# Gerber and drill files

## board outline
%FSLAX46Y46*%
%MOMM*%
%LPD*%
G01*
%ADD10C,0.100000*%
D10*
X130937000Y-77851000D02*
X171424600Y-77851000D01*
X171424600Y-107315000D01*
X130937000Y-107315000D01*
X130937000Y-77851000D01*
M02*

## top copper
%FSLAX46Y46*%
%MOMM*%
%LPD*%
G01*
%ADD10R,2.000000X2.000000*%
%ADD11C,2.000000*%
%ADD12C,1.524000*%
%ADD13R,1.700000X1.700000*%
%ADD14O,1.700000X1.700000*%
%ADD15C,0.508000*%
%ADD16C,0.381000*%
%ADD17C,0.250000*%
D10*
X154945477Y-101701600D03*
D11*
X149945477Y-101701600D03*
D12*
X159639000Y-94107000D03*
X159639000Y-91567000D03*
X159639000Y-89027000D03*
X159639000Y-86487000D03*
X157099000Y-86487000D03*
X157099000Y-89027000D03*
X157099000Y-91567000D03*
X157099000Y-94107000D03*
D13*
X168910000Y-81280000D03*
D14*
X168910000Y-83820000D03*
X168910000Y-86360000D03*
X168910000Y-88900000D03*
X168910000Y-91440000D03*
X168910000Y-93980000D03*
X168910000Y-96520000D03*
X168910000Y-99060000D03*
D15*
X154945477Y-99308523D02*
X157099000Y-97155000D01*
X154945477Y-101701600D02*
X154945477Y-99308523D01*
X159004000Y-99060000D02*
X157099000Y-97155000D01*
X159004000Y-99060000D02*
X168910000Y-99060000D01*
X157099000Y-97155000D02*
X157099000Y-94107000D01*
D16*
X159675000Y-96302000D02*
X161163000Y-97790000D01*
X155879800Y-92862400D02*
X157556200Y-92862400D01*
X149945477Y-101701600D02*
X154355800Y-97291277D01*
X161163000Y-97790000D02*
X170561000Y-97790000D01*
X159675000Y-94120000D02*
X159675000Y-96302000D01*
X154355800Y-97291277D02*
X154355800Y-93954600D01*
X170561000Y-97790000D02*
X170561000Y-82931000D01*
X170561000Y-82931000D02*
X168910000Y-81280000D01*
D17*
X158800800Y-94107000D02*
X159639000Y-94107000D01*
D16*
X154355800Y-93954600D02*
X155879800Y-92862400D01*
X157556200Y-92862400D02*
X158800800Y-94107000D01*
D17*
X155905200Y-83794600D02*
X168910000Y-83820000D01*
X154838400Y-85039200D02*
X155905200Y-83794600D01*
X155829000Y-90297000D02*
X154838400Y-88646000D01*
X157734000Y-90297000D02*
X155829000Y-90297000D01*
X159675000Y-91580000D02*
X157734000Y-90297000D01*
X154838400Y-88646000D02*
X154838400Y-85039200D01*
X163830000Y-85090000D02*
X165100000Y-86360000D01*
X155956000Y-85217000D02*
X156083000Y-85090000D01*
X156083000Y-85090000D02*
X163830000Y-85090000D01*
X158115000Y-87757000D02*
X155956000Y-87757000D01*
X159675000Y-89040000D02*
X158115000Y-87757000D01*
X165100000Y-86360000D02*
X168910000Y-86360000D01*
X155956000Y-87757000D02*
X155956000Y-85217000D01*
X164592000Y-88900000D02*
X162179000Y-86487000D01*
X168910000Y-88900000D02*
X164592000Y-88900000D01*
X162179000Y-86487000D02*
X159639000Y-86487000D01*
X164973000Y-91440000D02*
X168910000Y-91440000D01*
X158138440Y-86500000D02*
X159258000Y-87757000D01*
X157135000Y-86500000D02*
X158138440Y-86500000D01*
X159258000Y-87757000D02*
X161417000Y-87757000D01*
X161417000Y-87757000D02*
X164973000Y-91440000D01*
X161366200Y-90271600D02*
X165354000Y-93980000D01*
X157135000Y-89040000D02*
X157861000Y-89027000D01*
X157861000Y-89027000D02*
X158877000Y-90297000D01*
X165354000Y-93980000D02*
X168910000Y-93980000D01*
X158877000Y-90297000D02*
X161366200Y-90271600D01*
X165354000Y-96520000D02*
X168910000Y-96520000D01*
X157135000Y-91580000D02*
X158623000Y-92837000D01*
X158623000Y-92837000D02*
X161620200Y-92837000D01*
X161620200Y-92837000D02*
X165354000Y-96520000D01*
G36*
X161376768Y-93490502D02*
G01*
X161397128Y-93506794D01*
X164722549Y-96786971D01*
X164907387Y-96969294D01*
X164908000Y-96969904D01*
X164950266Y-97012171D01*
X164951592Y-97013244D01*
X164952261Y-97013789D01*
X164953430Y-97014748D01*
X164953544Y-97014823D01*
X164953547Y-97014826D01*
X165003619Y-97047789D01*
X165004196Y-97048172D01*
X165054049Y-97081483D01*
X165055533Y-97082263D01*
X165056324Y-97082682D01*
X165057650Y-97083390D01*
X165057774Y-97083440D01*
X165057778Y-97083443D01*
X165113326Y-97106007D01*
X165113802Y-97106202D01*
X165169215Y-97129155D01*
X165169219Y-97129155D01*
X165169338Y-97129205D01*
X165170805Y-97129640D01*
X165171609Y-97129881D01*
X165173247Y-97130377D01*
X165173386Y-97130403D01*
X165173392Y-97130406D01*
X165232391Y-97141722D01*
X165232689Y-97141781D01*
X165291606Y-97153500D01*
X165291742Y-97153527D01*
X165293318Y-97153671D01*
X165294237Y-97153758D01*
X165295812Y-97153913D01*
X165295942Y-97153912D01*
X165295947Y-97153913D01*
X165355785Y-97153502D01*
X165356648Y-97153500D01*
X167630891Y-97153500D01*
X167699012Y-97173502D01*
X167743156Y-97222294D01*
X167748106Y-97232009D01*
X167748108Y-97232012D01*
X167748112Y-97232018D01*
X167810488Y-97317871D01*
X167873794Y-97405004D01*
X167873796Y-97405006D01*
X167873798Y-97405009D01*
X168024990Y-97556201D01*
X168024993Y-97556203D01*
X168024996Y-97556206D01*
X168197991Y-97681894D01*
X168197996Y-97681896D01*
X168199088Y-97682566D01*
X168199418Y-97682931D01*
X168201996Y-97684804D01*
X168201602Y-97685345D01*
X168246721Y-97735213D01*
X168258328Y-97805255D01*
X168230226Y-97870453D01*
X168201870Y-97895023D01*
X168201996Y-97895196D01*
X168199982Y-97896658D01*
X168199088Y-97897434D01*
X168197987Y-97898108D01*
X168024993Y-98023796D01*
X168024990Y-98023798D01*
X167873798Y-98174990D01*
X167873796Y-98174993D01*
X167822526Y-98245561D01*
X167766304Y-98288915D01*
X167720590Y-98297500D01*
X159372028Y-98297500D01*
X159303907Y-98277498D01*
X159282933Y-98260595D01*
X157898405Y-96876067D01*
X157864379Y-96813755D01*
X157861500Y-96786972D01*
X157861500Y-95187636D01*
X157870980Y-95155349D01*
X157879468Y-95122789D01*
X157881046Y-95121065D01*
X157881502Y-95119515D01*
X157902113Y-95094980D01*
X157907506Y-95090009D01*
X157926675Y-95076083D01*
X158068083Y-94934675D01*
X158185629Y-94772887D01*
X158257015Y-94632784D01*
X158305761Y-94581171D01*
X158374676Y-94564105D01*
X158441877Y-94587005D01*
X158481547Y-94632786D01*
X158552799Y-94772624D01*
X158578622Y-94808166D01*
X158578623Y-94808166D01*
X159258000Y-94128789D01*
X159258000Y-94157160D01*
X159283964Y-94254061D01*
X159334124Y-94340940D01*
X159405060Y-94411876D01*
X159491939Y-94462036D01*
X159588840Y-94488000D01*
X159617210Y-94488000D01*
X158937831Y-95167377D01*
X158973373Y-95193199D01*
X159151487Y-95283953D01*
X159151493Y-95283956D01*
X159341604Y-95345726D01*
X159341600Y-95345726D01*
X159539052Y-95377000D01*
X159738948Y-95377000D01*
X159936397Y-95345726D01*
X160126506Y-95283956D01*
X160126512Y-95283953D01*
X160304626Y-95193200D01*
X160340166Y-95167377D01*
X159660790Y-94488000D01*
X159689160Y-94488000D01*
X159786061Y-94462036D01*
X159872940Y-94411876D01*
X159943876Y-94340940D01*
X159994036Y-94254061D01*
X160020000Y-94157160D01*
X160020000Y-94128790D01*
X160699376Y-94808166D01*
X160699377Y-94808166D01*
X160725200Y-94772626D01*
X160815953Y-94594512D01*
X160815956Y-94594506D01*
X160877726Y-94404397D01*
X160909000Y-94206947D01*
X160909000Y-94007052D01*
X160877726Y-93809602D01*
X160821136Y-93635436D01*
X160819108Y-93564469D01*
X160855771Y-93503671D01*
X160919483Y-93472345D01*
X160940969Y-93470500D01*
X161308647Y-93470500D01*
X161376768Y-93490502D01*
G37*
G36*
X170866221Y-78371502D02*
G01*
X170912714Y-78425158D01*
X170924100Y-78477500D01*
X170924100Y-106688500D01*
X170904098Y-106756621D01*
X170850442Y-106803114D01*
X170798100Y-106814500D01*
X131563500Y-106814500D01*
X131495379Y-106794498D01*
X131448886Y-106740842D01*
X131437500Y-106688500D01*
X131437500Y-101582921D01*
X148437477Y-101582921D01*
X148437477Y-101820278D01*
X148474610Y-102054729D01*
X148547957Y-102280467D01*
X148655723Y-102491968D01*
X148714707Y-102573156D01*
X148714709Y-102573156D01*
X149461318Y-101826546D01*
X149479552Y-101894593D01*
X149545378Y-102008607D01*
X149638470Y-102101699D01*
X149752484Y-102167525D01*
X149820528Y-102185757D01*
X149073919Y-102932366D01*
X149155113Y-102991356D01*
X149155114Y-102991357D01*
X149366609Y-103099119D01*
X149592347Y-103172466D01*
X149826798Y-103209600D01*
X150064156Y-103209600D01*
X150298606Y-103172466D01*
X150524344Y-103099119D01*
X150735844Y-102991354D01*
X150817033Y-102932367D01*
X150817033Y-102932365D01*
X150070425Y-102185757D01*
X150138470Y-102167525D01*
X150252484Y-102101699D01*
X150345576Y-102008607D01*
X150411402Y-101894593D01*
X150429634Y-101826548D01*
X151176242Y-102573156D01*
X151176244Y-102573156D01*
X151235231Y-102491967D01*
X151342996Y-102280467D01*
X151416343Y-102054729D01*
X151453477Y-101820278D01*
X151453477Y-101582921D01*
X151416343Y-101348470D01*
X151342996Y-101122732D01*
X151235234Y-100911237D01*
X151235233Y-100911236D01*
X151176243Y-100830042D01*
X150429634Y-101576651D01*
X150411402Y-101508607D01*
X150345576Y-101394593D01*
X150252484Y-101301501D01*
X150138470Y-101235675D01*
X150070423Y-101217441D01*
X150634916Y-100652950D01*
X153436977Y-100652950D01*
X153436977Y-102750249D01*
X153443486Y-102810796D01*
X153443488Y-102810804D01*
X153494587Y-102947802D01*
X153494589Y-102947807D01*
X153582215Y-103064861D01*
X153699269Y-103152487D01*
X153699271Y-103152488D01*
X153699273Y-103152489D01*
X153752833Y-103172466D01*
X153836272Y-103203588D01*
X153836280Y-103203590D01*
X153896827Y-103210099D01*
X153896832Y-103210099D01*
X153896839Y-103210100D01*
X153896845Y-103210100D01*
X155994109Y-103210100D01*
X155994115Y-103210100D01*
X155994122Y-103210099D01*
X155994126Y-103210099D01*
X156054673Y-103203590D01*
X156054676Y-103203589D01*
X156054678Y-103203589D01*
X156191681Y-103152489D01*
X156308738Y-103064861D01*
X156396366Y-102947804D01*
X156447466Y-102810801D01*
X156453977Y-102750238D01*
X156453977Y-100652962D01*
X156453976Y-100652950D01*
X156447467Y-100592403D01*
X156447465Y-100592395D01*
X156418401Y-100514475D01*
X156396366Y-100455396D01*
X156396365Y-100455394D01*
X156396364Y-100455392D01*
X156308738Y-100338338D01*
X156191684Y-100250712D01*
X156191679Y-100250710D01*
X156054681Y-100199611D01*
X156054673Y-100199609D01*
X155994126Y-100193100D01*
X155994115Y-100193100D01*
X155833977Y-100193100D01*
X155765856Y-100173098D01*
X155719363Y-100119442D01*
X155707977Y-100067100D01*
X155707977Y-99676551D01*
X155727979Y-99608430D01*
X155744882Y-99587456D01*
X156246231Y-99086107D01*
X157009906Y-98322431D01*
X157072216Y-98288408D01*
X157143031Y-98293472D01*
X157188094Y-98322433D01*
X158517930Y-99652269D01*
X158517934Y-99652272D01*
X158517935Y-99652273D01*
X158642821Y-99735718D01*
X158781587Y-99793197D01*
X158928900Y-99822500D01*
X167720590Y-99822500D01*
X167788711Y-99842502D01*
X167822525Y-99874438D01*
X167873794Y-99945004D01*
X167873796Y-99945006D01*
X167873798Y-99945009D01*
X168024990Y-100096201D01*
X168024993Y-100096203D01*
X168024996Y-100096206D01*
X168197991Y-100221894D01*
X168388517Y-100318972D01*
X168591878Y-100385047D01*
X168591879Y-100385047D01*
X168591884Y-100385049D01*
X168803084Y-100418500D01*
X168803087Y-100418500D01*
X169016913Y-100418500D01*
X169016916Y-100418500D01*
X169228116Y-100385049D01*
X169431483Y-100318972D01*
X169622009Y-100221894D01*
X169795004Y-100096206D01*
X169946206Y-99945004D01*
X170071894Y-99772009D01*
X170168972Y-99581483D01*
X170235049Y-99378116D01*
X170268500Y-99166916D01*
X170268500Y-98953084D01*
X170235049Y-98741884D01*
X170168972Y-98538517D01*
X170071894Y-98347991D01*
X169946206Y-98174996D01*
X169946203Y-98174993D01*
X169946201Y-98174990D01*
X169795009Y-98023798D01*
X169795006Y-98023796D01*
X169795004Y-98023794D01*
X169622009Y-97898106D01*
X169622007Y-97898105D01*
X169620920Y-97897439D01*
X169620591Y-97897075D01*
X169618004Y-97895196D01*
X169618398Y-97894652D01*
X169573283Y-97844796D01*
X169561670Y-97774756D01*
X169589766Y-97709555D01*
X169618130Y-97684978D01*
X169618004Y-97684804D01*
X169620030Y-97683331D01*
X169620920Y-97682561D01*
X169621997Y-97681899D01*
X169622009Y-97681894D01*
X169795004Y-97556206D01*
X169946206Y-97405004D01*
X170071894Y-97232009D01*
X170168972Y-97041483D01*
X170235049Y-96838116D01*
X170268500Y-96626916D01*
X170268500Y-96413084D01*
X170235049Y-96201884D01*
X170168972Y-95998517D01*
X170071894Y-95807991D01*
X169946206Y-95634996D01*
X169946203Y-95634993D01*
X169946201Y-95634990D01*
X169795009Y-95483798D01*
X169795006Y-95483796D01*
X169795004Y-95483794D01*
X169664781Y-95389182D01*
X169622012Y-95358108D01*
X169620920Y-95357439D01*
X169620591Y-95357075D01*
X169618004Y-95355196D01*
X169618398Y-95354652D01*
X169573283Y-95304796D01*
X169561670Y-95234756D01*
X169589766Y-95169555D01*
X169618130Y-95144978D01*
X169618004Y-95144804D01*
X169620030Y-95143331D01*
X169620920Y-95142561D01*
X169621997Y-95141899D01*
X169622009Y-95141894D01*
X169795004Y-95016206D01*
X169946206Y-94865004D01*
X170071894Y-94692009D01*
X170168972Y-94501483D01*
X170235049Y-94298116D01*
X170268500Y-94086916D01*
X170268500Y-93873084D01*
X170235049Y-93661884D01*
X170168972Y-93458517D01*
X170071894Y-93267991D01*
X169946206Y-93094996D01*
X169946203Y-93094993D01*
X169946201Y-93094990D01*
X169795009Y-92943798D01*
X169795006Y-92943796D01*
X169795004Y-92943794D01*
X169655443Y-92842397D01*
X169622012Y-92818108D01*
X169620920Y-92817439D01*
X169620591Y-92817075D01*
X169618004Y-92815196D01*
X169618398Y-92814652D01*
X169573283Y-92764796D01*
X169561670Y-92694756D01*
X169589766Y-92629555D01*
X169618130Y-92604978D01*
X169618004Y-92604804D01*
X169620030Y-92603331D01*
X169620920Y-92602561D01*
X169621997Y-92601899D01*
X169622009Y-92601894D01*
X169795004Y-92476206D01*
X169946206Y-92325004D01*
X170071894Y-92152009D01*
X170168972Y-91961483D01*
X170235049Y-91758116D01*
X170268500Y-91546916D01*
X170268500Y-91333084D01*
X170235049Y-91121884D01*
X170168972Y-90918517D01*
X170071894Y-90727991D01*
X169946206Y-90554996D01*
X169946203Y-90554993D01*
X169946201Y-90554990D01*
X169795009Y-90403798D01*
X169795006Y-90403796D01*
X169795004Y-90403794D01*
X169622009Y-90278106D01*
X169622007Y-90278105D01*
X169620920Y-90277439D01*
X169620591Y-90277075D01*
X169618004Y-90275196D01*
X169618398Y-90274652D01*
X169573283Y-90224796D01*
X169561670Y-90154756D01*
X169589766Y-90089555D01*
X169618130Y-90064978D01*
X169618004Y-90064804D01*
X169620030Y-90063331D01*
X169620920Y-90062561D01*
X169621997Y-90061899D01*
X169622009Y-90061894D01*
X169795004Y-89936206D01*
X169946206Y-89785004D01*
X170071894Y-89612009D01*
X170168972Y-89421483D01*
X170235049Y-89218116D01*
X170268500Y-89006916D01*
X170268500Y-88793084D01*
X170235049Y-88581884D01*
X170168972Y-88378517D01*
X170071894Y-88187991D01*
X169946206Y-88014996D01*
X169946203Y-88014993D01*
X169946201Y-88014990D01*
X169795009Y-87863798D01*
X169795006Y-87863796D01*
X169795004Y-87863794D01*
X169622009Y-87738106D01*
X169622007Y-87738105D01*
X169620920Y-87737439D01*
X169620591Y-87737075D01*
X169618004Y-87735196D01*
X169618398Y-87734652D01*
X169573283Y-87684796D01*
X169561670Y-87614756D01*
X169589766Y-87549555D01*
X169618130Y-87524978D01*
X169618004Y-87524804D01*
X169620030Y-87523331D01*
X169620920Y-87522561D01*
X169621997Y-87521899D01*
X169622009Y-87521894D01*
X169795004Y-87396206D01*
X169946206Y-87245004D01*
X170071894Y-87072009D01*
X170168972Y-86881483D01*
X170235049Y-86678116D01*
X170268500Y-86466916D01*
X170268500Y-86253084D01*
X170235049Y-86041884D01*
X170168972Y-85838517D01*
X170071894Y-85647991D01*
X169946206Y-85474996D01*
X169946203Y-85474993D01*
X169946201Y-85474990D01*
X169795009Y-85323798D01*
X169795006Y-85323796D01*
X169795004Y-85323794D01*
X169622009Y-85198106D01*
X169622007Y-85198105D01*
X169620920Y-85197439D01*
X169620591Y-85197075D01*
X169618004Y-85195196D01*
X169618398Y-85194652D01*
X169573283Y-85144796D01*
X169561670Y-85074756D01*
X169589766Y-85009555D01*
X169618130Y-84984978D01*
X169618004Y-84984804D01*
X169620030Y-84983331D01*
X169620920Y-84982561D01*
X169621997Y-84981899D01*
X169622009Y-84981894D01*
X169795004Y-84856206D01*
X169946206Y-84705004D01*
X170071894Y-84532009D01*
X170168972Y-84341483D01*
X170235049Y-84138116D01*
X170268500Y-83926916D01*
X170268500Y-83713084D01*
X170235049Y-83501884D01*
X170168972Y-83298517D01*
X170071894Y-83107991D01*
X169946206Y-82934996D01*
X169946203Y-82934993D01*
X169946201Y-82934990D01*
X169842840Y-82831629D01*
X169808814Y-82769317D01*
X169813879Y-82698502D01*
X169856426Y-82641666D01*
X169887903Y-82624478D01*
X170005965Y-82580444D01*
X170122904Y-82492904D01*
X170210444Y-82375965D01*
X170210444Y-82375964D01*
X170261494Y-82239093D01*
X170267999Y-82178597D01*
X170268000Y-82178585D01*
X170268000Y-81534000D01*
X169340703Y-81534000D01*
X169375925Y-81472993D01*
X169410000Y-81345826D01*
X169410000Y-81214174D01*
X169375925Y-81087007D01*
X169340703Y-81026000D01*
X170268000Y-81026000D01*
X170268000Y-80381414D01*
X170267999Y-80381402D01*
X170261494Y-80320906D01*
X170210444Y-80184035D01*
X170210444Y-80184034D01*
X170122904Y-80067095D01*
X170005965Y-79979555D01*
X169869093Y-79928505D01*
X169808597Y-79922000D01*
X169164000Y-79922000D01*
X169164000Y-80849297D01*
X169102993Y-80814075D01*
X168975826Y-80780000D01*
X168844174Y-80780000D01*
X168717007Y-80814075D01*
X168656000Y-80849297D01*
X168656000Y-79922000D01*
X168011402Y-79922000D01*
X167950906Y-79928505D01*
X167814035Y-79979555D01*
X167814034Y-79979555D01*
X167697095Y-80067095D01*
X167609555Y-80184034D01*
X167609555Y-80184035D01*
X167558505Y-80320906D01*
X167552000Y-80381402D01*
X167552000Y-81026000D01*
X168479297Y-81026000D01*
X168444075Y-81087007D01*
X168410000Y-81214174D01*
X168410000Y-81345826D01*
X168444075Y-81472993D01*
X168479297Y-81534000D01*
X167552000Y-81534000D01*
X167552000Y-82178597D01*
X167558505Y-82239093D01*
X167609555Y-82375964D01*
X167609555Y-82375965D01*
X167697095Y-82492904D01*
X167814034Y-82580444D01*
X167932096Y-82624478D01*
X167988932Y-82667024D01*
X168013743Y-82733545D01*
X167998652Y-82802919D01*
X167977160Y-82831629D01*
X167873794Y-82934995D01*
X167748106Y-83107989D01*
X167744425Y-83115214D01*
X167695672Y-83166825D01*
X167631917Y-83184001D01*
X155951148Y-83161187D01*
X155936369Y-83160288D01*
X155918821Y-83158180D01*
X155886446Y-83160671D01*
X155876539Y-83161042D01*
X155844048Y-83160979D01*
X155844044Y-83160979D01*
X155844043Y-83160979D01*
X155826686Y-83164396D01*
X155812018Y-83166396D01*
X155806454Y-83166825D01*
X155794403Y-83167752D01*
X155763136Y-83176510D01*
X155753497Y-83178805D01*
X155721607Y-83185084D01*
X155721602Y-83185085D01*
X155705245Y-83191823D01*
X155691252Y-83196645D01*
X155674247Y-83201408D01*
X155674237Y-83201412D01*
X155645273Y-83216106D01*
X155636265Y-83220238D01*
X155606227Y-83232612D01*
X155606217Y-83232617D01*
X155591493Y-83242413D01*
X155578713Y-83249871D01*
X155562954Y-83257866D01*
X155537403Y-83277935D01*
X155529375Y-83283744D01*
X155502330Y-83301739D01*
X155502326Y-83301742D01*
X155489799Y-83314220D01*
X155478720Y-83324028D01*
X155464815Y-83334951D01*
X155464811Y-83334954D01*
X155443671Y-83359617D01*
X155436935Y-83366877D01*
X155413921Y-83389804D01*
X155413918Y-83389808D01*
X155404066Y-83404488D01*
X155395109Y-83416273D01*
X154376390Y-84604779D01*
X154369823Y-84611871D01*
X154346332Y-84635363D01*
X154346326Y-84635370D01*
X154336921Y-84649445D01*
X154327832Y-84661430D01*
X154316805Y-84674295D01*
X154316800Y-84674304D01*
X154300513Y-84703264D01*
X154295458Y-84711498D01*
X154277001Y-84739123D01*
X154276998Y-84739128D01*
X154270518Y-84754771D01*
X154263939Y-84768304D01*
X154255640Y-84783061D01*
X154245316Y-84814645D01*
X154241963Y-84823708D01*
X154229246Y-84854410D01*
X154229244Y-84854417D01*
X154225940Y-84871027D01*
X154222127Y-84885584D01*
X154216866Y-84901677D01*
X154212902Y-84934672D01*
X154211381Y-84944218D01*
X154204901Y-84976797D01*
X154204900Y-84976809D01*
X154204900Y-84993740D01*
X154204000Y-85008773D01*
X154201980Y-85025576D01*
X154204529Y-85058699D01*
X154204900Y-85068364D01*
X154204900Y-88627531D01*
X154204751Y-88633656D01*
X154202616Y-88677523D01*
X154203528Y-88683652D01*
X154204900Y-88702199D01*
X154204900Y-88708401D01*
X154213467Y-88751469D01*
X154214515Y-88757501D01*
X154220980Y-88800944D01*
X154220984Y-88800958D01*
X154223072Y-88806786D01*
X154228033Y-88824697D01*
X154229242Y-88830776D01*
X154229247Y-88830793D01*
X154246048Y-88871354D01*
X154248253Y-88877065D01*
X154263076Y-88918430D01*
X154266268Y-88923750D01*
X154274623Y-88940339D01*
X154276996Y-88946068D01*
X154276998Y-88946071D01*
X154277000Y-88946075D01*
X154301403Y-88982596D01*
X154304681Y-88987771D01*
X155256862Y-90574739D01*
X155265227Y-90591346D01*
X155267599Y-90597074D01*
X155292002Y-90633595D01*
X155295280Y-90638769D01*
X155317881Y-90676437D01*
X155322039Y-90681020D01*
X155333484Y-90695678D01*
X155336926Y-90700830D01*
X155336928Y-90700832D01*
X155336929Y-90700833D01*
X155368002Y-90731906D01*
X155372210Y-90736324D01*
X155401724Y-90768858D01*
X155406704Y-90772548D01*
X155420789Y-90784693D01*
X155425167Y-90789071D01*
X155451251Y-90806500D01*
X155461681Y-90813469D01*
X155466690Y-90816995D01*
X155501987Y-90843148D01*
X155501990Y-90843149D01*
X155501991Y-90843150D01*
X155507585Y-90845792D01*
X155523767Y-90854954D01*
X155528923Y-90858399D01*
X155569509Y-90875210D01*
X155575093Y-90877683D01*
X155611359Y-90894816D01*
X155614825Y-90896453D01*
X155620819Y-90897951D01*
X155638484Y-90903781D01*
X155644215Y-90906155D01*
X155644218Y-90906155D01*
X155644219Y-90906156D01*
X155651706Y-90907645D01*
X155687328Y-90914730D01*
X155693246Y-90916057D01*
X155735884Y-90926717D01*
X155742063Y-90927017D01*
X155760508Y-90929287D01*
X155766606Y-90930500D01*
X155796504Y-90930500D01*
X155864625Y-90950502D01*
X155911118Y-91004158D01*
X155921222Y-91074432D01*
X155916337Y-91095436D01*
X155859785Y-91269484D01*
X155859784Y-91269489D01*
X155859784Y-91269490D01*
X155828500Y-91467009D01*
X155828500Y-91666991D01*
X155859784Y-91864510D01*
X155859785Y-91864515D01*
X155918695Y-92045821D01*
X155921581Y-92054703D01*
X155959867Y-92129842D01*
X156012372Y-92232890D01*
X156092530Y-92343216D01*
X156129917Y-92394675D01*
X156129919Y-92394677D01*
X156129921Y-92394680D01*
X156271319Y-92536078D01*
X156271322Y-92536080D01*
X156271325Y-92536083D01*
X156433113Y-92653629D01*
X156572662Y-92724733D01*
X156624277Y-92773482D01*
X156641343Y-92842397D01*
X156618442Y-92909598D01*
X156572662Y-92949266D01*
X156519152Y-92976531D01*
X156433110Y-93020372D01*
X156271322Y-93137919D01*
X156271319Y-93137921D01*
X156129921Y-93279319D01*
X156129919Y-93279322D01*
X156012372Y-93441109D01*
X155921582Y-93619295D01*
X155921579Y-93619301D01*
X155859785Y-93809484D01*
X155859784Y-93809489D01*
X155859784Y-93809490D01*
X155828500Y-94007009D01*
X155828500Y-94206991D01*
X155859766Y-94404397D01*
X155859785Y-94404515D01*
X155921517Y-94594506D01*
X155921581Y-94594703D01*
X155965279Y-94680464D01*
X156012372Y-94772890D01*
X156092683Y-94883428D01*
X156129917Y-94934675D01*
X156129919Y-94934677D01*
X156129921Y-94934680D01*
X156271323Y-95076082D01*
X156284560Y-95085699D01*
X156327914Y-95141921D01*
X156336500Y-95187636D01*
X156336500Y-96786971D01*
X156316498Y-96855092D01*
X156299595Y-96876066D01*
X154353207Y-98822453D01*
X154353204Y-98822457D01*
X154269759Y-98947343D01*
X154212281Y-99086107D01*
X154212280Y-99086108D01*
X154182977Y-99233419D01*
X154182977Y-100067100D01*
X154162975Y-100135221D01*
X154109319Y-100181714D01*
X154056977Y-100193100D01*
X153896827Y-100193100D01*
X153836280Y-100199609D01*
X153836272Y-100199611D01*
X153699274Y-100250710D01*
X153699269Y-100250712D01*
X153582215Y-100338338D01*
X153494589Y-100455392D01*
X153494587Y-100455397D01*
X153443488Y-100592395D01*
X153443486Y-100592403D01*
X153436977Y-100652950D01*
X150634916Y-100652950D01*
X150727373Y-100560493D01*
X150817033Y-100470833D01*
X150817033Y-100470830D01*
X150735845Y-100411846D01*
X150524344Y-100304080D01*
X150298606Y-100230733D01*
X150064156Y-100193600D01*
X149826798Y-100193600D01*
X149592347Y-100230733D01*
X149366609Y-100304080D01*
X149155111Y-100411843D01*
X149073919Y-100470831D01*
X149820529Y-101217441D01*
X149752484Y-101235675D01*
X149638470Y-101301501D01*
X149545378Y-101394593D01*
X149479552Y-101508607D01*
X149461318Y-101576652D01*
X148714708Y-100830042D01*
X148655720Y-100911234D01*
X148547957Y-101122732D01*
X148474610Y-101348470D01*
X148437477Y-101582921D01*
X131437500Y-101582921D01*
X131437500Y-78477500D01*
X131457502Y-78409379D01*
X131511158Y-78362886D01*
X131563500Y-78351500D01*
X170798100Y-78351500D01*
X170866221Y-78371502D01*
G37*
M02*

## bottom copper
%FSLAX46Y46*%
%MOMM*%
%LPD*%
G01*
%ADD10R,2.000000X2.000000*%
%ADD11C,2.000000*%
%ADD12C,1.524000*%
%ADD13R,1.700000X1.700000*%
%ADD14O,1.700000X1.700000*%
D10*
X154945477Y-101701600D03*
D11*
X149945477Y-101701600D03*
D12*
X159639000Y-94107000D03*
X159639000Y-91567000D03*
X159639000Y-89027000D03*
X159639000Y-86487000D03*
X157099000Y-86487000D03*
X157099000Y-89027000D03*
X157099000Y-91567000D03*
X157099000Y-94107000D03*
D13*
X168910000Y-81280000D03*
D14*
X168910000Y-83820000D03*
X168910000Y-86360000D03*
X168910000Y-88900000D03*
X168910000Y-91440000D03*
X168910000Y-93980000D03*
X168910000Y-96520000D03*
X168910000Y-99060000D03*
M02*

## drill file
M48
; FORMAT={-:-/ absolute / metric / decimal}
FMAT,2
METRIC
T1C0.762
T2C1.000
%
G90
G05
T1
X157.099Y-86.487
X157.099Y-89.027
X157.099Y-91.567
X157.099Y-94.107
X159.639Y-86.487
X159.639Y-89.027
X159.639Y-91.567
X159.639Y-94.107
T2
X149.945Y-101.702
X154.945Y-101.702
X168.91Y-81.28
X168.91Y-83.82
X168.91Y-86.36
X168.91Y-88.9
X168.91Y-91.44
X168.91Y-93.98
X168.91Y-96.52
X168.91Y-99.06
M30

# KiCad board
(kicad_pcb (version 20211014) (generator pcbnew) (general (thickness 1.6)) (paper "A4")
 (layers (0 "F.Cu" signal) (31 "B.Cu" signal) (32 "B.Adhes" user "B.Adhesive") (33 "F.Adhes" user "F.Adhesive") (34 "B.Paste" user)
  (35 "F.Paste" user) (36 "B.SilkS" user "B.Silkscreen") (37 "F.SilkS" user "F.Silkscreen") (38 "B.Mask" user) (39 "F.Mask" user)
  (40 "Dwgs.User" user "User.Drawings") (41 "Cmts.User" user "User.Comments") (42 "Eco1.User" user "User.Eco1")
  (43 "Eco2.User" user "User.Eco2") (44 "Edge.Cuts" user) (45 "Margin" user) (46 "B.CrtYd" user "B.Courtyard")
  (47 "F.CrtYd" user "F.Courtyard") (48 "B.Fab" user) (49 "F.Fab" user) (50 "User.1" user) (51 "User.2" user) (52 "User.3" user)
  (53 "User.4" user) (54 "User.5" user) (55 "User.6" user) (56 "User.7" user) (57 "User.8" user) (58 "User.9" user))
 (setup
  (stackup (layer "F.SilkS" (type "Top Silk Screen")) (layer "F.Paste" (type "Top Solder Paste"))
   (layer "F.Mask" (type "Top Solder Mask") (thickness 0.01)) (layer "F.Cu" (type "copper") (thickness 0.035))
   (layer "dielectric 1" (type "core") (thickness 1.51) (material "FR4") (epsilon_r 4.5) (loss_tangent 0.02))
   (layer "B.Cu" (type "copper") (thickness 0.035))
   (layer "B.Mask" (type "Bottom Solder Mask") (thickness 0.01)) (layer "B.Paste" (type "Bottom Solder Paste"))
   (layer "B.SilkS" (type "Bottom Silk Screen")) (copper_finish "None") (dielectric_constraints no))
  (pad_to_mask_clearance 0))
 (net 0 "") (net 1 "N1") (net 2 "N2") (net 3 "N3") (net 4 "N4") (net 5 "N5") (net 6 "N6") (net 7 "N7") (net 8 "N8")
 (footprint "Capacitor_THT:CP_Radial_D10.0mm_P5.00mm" (layer "F.Cu") (at 154.945477 101.7016 180)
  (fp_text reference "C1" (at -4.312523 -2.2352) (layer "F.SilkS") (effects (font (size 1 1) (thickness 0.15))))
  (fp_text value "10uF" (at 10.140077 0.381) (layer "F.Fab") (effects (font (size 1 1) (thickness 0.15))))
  (pad "1" thru_hole rect (at 0 0 180) (size 2 2) (drill 1) (layers *.Cu *.Mask) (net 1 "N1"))
  (pad "2" thru_hole circle (at 5 0 180) (size 2 2) (drill 1) (layers *.Cu *.Mask) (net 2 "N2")))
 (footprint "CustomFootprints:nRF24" (layer "F.Cu") (at 153.289 90.932)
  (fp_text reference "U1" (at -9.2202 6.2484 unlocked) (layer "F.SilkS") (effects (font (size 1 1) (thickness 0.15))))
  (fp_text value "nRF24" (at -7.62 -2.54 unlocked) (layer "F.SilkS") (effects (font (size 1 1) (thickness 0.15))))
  (pad "0" thru_hole circle (at 6.35 3.175) (size 1.524 1.524) (drill 0.762) (layers *.Cu *.Mask) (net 2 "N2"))
  (pad "1" thru_hole circle (at 6.35 0.635) (size 1.524 1.524) (drill 0.762) (layers *.Cu *.Mask) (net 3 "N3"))
  (pad "2" thru_hole circle (at 6.35 -1.905) (size 1.524 1.524) (drill 0.762) (layers *.Cu *.Mask) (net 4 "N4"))
  (pad "3" thru_hole circle (at 6.35 -4.445) (size 1.524 1.524) (drill 0.762) (layers *.Cu *.Mask) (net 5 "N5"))
  (pad "4" thru_hole circle (at 3.81 -4.445) (size 1.524 1.524) (drill 0.762) (layers *.Cu *.Mask) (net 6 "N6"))
  (pad "5" thru_hole circle (at 3.81 -1.905) (size 1.524 1.524) (drill 0.762) (layers *.Cu *.Mask) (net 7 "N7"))
  (pad "6" thru_hole circle (at 3.81 0.635) (size 1.524 1.524) (drill 0.762) (layers *.Cu *.Mask) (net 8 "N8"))
  (pad "7" thru_hole circle (at 3.81 3.175) (size 1.524 1.524) (drill 0.762) (layers *.Cu *.Mask) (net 1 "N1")))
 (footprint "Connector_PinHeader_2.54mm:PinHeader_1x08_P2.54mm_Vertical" (layer "B.Cu") (at 168.91 81.28 180)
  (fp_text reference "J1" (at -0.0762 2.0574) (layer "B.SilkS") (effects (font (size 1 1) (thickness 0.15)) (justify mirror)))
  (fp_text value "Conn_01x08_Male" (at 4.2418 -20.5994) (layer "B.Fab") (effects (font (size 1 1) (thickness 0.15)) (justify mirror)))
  (pad "1" thru_hole rect (at 0 0 180) (size 1.7 1.7) (drill 1) (layers *.Cu *.Mask) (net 2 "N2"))
  (pad "2" thru_hole oval (at 0 -2.54 180) (size 1.7 1.7) (drill 1) (layers *.Cu *.Mask) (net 3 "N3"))
  (pad "3" thru_hole oval (at 0 -5.08 180) (size 1.7 1.7) (drill 1) (layers *.Cu *.Mask) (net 4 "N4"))
  (pad "4" thru_hole oval (at 0 -7.62 180) (size 1.7 1.7) (drill 1) (layers *.Cu *.Mask) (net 5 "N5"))
  (pad "5" thru_hole oval (at 0 -10.16 180) (size 1.7 1.7) (drill 1) (layers *.Cu *.Mask) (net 6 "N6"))
  (pad "6" thru_hole oval (at 0 -12.7 180) (size 1.7 1.7) (drill 1) (layers *.Cu *.Mask) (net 7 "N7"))
  (pad "7" thru_hole oval (at 0 -15.24 180) (size 1.7 1.7) (drill 1) (layers *.Cu *.Mask) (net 8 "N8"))
  (pad "8" thru_hole oval (at 0 -17.78 180) (size 1.7 1.7) (drill 1) (layers *.Cu *.Mask) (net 1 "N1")))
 (gr_rect (start 130.937 77.851) (end 171.4246 107.315) (layer "Edge.Cuts") (width 0.1) (fill none))
 (segment (start 154.945477 99.308523) (end 157.099 97.155) (width 0.508) (layer "F.Cu") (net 1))
 (segment (start 154.945477 101.7016) (end 154.945477 99.308523) (width 0.508) (layer "F.Cu") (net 1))
 (segment (start 159.004 99.06) (end 157.099 97.155) (width 0.508) (layer "F.Cu") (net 1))
 (segment (start 159.004 99.06) (end 168.91 99.06) (width 0.508) (layer "F.Cu") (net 1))
 (segment (start 157.099 97.155) (end 157.099 94.107) (width 0.508) (layer "F.Cu") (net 1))
 (segment (start 159.675 96.302) (end 161.163 97.79) (width 0.381) (layer "F.Cu") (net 2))
 (segment (start 155.8798 92.8624) (end 157.5562 92.8624) (width 0.381) (layer "F.Cu") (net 2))
 (segment (start 149.945477 101.7016) (end 154.3558 97.291277) (width 0.381) (layer "F.Cu") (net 2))
 (segment (start 161.163 97.79) (end 170.561 97.79) (width 0.381) (layer "F.Cu") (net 2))
 (segment (start 159.675 94.12) (end 159.675 96.302) (width 0.381) (layer "F.Cu") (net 2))
 (segment (start 154.3558 97.291277) (end 154.3558 93.9546) (width 0.381) (layer "F.Cu") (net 2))
 (segment (start 170.561 97.79) (end 170.561 82.931) (width 0.381) (layer "F.Cu") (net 2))
 (segment (start 170.561 82.931) (end 168.91 81.28) (width 0.381) (layer "F.Cu") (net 2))
 (segment (start 158.8008 94.107) (end 159.639 94.107) (width 0.25) (layer "F.Cu") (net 2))
 (segment (start 154.3558 93.9546) (end 155.8798 92.8624) (width 0.381) (layer "F.Cu") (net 2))
 (segment (start 157.5562 92.8624) (end 158.8008 94.107) (width 0.381) (layer "F.Cu") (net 2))
 (segment (start 155.9052 83.7946) (end 168.91 83.82) (width 0.25) (layer "F.Cu") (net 3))
 (segment (start 154.8384 85.0392) (end 155.9052 83.7946) (width 0.25) (layer "F.Cu") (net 3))
 (segment (start 155.829 90.297) (end 154.8384 88.646) (width 0.25) (layer "F.Cu") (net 3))
 (segment (start 157.734 90.297) (end 155.829 90.297) (width 0.25) (layer "F.Cu") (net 3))
 (segment (start 159.675 91.58) (end 157.734 90.297) (width 0.25) (layer "F.Cu") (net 3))
 (segment (start 154.8384 88.646) (end 154.8384 85.0392) (width 0.25) (layer "F.Cu") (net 3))
 (segment (start 163.83 85.09) (end 165.1 86.36) (width 0.25) (layer "F.Cu") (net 4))
 (segment (start 155.956 85.217) (end 156.083 85.09) (width 0.25) (layer "F.Cu") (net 4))
 (segment (start 156.083 85.09) (end 163.83 85.09) (width 0.25) (layer "F.Cu") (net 4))
 (segment (start 158.115 87.757) (end 155.956 87.757) (width 0.25) (layer "F.Cu") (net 4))
 (segment (start 159.675 89.04) (end 158.115 87.757) (width 0.25) (layer "F.Cu") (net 4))
 (segment (start 165.1 86.36) (end 168.91 86.36) (width 0.25) (layer "F.Cu") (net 4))
 (segment (start 155.956 87.757) (end 155.956 85.217) (width 0.25) (layer "F.Cu") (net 4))
 (segment (start 164.592 88.9) (end 162.179 86.487) (width 0.25) (layer "F.Cu") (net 5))
 (segment (start 168.91 88.9) (end 164.592 88.9) (width 0.25) (layer "F.Cu") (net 5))
 (segment (start 162.179 86.487) (end 159.639 86.487) (width 0.25) (layer "F.Cu") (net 5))
 (segment (start 164.973 91.44) (end 168.91 91.44) (width 0.25) (layer "F.Cu") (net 6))
 (segment (start 158.13844 86.5) (end 159.258 87.757) (width 0.25) (layer "F.Cu") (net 6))
 (segment (start 157.135 86.5) (end 158.13844 86.5) (width 0.25) (layer "F.Cu") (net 6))
 (segment (start 159.258 87.757) (end 161.417 87.757) (width 0.25) (layer "F.Cu") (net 6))
 (segment (start 161.417 87.757) (end 164.973 91.44) (width 0.25) (layer "F.Cu") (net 6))
 (segment (start 161.3662 90.2716) (end 165.354 93.98) (width 0.25) (layer "F.Cu") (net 7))
 (segment (start 157.135 89.04) (end 157.861 89.027) (width 0.25) (layer "F.Cu") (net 7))
 (segment (start 157.861 89.027) (end 158.877 90.297) (width 0.25) (layer "F.Cu") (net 7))
 (segment (start 165.354 93.98) (end 168.91 93.98) (width 0.25) (layer "F.Cu") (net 7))
 (segment (start 158.877 90.297) (end 161.3662 90.2716) (width 0.25) (layer "F.Cu") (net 7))
 (segment (start 165.354 96.52) (end 168.91 96.52) (width 0.25) (layer "F.Cu") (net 8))
 (segment (start 157.135 91.58) (end 158.623 92.837) (width 0.25) (layer "F.Cu") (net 8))
 (segment (start 158.623 92.837) (end 161.6202 92.837) (width 0.25) (layer "F.Cu") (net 8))
 (segment (start 161.6202 92.837) (end 165.354 96.52) (width 0.25) (layer "F.Cu") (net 8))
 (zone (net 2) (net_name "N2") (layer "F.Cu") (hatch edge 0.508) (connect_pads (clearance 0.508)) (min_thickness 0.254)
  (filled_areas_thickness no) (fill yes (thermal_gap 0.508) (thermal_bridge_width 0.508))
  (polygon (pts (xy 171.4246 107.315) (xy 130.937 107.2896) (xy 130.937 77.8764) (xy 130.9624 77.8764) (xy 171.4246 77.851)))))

